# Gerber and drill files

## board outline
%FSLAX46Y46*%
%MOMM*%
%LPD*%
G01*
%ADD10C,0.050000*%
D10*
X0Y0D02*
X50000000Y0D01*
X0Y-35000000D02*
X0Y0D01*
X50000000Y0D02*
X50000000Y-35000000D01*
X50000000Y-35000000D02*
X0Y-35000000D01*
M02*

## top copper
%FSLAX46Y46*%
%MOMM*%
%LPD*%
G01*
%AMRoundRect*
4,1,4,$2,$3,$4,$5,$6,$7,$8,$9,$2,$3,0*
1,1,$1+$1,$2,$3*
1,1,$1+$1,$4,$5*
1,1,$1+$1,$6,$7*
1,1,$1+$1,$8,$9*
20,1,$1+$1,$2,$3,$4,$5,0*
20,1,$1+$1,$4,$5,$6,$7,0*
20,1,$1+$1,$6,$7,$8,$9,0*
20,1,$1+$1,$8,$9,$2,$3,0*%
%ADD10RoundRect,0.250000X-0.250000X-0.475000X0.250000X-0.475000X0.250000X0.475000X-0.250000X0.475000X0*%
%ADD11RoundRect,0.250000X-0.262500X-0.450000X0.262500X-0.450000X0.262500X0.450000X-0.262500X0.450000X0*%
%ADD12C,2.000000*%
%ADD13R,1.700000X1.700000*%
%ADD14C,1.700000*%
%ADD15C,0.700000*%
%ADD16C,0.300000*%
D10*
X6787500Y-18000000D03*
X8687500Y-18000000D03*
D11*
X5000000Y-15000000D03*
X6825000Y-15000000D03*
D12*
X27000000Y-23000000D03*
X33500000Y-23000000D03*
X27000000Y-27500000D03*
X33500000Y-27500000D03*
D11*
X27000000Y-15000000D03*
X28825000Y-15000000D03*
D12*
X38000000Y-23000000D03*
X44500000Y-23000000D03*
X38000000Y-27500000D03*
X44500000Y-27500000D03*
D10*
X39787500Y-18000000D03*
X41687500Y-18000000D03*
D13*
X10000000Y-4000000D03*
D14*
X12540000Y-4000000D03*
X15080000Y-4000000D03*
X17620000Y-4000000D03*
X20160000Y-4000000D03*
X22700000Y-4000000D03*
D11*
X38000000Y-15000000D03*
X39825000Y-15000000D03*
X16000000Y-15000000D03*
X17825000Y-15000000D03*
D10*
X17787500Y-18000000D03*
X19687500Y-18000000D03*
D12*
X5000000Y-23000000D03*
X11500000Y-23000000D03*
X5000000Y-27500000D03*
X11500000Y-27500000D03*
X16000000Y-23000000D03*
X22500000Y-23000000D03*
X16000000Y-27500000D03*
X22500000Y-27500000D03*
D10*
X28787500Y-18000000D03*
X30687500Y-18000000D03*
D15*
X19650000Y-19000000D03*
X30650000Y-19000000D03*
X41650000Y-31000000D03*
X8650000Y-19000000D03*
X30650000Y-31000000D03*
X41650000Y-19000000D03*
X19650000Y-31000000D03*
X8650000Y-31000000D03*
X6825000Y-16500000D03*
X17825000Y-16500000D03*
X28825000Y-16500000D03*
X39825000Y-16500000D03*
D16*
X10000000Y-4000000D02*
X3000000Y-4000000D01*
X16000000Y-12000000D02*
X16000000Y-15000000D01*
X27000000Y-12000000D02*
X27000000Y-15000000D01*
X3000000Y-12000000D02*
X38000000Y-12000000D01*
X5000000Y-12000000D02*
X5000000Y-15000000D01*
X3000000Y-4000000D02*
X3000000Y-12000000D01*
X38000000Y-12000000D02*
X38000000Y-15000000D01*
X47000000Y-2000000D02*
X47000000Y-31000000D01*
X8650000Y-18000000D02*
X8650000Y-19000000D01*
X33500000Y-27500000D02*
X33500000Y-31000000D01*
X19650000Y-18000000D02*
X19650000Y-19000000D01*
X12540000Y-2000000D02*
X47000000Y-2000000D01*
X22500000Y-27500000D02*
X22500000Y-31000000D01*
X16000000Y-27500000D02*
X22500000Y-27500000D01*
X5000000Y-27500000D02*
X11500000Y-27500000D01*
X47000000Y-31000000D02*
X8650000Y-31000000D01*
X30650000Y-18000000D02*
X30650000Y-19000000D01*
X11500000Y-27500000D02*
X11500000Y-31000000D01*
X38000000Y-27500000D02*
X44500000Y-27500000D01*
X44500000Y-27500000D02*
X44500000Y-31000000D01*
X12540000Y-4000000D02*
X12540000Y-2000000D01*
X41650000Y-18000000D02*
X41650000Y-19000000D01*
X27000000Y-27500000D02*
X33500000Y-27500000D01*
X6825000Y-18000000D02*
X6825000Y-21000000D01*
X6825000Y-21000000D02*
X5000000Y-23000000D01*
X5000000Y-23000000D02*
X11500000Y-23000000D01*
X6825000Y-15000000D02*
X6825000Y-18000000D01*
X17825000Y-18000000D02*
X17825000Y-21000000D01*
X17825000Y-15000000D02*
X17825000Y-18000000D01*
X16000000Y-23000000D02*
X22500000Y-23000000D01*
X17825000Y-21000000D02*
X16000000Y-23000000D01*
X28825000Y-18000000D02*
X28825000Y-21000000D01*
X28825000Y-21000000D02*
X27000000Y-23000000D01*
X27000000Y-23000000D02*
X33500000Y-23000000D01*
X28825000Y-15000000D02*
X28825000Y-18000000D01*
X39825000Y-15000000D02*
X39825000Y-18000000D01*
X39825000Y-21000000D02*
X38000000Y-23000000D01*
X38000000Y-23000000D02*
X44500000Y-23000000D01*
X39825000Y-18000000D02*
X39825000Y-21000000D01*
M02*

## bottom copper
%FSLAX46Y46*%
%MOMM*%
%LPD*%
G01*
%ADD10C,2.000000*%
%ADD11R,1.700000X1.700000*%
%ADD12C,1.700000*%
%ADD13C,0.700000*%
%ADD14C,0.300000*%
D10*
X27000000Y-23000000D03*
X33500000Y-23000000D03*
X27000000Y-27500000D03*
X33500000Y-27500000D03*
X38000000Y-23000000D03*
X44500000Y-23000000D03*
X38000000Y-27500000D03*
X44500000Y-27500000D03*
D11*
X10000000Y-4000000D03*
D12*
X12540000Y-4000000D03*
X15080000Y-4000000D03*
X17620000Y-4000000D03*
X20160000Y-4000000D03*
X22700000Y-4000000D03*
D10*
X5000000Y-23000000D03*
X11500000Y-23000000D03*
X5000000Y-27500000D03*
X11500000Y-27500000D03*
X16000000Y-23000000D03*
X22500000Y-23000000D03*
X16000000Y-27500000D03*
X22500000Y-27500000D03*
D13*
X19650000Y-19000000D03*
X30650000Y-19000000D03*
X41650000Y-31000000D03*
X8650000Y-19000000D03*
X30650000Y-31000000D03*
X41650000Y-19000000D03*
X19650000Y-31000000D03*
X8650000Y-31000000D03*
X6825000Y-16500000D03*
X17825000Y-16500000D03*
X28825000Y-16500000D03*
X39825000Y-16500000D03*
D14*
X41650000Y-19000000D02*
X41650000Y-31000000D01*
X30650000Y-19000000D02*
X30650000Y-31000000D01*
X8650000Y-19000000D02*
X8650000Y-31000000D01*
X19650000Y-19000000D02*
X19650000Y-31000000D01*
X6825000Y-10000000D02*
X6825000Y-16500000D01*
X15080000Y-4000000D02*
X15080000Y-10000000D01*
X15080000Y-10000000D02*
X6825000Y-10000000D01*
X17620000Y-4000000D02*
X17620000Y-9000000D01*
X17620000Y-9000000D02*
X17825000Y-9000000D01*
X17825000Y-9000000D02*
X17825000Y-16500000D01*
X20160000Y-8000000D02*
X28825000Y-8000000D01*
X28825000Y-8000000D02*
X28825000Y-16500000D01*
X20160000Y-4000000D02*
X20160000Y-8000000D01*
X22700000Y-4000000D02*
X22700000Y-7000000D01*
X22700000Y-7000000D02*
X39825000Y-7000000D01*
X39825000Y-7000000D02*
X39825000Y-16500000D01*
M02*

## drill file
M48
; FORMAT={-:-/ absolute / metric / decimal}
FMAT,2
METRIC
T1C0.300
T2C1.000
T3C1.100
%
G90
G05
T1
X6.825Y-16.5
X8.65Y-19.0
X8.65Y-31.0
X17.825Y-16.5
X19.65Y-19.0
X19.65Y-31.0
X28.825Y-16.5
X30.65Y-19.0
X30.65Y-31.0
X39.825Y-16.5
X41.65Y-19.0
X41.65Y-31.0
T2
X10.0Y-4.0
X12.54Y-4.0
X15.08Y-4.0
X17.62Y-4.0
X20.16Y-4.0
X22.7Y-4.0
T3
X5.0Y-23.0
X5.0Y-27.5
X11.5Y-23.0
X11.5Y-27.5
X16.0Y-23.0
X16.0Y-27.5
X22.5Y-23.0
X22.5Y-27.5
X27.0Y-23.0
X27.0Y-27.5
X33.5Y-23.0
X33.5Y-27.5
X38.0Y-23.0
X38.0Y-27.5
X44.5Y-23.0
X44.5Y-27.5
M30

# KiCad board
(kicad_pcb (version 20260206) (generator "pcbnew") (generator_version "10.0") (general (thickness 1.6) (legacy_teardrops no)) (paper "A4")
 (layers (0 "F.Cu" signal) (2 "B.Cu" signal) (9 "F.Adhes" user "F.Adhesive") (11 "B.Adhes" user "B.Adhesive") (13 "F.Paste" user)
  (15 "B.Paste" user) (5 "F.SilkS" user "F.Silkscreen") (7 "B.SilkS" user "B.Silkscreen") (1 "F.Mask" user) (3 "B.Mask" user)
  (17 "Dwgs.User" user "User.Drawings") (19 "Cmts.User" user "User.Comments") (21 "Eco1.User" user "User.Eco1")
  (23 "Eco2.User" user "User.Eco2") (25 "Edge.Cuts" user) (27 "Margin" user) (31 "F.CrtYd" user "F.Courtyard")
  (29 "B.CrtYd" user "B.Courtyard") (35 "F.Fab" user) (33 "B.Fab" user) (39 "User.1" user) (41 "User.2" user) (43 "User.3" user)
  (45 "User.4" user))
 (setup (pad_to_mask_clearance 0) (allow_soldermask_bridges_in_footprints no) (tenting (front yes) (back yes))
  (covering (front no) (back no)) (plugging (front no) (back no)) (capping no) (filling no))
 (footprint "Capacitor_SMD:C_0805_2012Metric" (layer "F.Cu") (at 7.7375 18)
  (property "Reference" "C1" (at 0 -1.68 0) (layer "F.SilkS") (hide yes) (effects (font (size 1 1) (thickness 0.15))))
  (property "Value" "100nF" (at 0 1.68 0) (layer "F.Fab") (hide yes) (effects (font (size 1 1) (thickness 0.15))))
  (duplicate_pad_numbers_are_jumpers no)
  (pad "1" smd roundrect (at -0.95 0) (size 1 1.45) (layers "F.Cu" "F.Mask" "F.Paste") (roundrect_rratio 0.25) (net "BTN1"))
  (pad "2" smd roundrect (at 0.95 0) (size 1 1.45) (layers "F.Cu" "F.Mask" "F.Paste") (roundrect_rratio 0.25) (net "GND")))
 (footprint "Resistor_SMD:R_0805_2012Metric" (layer "F.Cu") (at 5.9125 15)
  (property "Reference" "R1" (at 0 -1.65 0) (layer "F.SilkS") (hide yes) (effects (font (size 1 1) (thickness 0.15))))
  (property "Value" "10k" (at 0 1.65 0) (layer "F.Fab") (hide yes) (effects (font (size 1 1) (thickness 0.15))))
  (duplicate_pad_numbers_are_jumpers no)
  (pad "1" smd roundrect (at -0.9125 0) (size 1.025 1.4) (layers "F.Cu" "F.Mask" "F.Paste") (roundrect_rratio 0.243902) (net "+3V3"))
  (pad "2" smd roundrect (at 0.9125 0) (size 1.025 1.4) (layers "F.Cu" "F.Mask" "F.Paste") (roundrect_rratio 0.243902) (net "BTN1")))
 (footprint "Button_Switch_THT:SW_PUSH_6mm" (layer "F.Cu") (at 27 23)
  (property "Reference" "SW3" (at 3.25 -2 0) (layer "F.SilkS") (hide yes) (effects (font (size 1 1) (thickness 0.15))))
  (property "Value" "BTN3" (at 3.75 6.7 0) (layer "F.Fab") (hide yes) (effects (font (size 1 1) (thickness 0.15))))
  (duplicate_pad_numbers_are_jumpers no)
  (pad "1" thru_hole circle (at 0 0 90) (size 2 2) (drill 1.1) (layers "*.Cu" "*.Mask") (remove_unused_layers no) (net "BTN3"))
  (pad "1" thru_hole circle (at 6.5 0 90) (size 2 2) (drill 1.1) (layers "*.Cu" "*.Mask") (remove_unused_layers no) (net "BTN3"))
  (pad "2" thru_hole circle (at 0 4.5 90) (size 2 2) (drill 1.1) (layers "*.Cu" "*.Mask") (remove_unused_layers no) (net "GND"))
  (pad "2" thru_hole circle (at 6.5 4.5 90) (size 2 2) (drill 1.1) (layers "*.Cu" "*.Mask") (remove_unused_layers no) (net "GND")))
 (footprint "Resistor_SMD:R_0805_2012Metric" (layer "F.Cu") (at 27.9125 15)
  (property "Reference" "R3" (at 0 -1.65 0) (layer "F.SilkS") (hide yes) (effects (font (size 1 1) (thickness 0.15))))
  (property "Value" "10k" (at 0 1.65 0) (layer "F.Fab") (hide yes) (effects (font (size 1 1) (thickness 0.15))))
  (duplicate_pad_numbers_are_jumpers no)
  (pad "1" smd roundrect (at -0.9125 0) (size 1.025 1.4) (layers "F.Cu" "F.Mask" "F.Paste") (roundrect_rratio 0.243902) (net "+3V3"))
  (pad "2" smd roundrect (at 0.9125 0) (size 1.025 1.4) (layers "F.Cu" "F.Mask" "F.Paste") (roundrect_rratio 0.243902) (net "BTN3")))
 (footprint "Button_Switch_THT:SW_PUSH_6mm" (layer "F.Cu") (at 38 23)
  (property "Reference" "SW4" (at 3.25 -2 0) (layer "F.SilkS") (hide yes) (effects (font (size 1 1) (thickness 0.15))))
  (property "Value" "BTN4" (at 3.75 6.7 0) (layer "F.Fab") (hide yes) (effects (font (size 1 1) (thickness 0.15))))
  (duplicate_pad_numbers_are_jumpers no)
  (pad "1" thru_hole circle (at 0 0 90) (size 2 2) (drill 1.1) (layers "*.Cu" "*.Mask") (remove_unused_layers no) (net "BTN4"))
  (pad "1" thru_hole circle (at 6.5 0 90) (size 2 2) (drill 1.1) (layers "*.Cu" "*.Mask") (remove_unused_layers no) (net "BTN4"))
  (pad "2" thru_hole circle (at 0 4.5 90) (size 2 2) (drill 1.1) (layers "*.Cu" "*.Mask") (remove_unused_layers no) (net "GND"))
  (pad "2" thru_hole circle (at 6.5 4.5 90) (size 2 2) (drill 1.1) (layers "*.Cu" "*.Mask") (remove_unused_layers no) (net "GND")))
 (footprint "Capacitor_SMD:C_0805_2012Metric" (layer "F.Cu") (at 40.7375 18)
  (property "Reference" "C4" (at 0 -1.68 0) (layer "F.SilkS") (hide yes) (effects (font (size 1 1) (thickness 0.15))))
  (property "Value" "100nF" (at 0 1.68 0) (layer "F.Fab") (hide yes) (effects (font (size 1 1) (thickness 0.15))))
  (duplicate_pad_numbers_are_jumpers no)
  (pad "1" smd roundrect (at -0.95 0) (size 1 1.45) (layers "F.Cu" "F.Mask" "F.Paste") (roundrect_rratio 0.25) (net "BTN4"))
  (pad "2" smd roundrect (at 0.95 0) (size 1 1.45) (layers "F.Cu" "F.Mask" "F.Paste") (roundrect_rratio 0.25) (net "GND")))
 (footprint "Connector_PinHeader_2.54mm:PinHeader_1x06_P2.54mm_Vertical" (layer "F.Cu") (at 10 4 90)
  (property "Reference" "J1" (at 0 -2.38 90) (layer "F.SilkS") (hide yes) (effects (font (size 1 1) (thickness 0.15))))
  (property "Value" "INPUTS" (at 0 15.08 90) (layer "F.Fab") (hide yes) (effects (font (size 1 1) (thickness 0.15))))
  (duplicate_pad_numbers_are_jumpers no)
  (pad "1" thru_hole rect (at 0 0 90) (size 1.7 1.7) (drill 1) (layers "*.Cu" "*.Mask") (remove_unused_layers no) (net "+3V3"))
  (pad "2" thru_hole circle (at 0 2.54 90) (size 1.7 1.7) (drill 1) (layers "*.Cu" "*.Mask") (remove_unused_layers no) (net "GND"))
  (pad "3" thru_hole circle (at 0 5.08 90) (size 1.7 1.7) (drill 1) (layers "*.Cu" "*.Mask") (remove_unused_layers no) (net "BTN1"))
  (pad "4" thru_hole circle (at 0 7.62 90) (size 1.7 1.7) (drill 1) (layers "*.Cu" "*.Mask") (remove_unused_layers no) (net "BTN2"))
  (pad "5" thru_hole circle (at 0 10.16 90) (size 1.7 1.7) (drill 1) (layers "*.Cu" "*.Mask") (remove_unused_layers no) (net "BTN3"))
  (pad "6" thru_hole circle (at 0 12.7 90) (size 1.7 1.7) (drill 1) (layers "*.Cu" "*.Mask") (remove_unused_layers no) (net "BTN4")))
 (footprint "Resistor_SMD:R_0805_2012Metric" (layer "F.Cu") (at 38.9125 15)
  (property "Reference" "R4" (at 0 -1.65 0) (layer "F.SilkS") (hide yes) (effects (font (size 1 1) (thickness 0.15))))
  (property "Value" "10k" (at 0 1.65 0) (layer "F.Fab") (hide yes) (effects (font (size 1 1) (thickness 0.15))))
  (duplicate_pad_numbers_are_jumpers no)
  (pad "1" smd roundrect (at -0.9125 0) (size 1.025 1.4) (layers "F.Cu" "F.Mask" "F.Paste") (roundrect_rratio 0.243902) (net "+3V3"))
  (pad "2" smd roundrect (at 0.9125 0) (size 1.025 1.4) (layers "F.Cu" "F.Mask" "F.Paste") (roundrect_rratio 0.243902) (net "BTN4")))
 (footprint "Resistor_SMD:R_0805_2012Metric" (layer "F.Cu") (at 16.9125 15)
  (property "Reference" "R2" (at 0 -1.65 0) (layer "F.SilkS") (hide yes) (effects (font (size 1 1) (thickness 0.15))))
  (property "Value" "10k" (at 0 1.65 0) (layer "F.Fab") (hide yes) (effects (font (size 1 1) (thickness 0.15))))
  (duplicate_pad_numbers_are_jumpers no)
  (pad "1" smd roundrect (at -0.9125 0) (size 1.025 1.4) (layers "F.Cu" "F.Mask" "F.Paste") (roundrect_rratio 0.243902) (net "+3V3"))
  (pad "2" smd roundrect (at 0.9125 0) (size 1.025 1.4) (layers "F.Cu" "F.Mask" "F.Paste") (roundrect_rratio 0.243902) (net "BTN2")))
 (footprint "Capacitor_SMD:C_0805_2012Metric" (layer "F.Cu") (at 18.7375 18)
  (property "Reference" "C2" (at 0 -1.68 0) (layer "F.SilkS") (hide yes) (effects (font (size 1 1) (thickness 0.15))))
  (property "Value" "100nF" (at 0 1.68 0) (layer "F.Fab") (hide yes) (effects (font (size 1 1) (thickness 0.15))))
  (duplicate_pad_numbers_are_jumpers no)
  (pad "1" smd roundrect (at -0.95 0) (size 1 1.45) (layers "F.Cu" "F.Mask" "F.Paste") (roundrect_rratio 0.25) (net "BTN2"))
  (pad "2" smd roundrect (at 0.95 0) (size 1 1.45) (layers "F.Cu" "F.Mask" "F.Paste") (roundrect_rratio 0.25) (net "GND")))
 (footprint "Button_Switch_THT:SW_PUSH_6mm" (layer "F.Cu") (at 5 23)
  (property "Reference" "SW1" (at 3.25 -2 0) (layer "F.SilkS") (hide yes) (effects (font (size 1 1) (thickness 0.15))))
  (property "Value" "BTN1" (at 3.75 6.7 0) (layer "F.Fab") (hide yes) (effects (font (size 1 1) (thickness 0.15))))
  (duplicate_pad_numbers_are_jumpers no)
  (pad "1" thru_hole circle (at 0 0 90) (size 2 2) (drill 1.1) (layers "*.Cu" "*.Mask") (remove_unused_layers no) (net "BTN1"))
  (pad "1" thru_hole circle (at 6.5 0 90) (size 2 2) (drill 1.1) (layers "*.Cu" "*.Mask") (remove_unused_layers no) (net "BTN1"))
  (pad "2" thru_hole circle (at 0 4.5 90) (size 2 2) (drill 1.1) (layers "*.Cu" "*.Mask") (remove_unused_layers no) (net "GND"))
  (pad "2" thru_hole circle (at 6.5 4.5 90) (size 2 2) (drill 1.1) (layers "*.Cu" "*.Mask") (remove_unused_layers no) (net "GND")))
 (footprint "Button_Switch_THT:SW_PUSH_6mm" (layer "F.Cu") (at 16 23)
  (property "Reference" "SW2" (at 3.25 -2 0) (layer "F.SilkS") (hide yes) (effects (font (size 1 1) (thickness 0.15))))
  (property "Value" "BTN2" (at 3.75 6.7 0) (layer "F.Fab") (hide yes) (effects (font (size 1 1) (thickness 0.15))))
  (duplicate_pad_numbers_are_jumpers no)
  (pad "1" thru_hole circle (at 0 0 90) (size 2 2) (drill 1.1) (layers "*.Cu" "*.Mask") (remove_unused_layers no) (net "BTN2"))
  (pad "1" thru_hole circle (at 6.5 0 90) (size 2 2) (drill 1.1) (layers "*.Cu" "*.Mask") (remove_unused_layers no) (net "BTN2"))
  (pad "2" thru_hole circle (at 0 4.5 90) (size 2 2) (drill 1.1) (layers "*.Cu" "*.Mask") (remove_unused_layers no) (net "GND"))
  (pad "2" thru_hole circle (at 6.5 4.5 90) (size 2 2) (drill 1.1) (layers "*.Cu" "*.Mask") (remove_unused_layers no) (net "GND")))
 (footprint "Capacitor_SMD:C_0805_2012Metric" (layer "F.Cu") (at 29.7375 18)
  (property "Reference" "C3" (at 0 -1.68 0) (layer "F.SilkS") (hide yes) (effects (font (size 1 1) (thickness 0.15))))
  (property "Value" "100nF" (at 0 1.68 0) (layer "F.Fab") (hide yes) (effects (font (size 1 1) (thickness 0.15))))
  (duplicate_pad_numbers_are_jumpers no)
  (pad "1" smd roundrect (at -0.95 0) (size 1 1.45) (layers "F.Cu" "F.Mask" "F.Paste") (roundrect_rratio 0.25) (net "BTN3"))
  (pad "2" smd roundrect (at 0.95 0) (size 1 1.45) (layers "F.Cu" "F.Mask" "F.Paste") (roundrect_rratio 0.25) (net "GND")))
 (gr_line (start 0 0) (end 50 0) (stroke (width 0.05) (type default)) (layer "Edge.Cuts"))
 (gr_line (start 0 35) (end 0 0) (stroke (width 0.05) (type default)) (layer "Edge.Cuts"))
 (gr_line (start 50 0) (end 50 35) (stroke (width 0.05) (type default)) (layer "Edge.Cuts"))
 (gr_line (start 50 35) (end 0 35) (stroke (width 0.05) (type default)) (layer "Edge.Cuts"))
 (segment (start 10 4) (end 3 4) (width 0.3) (layer "F.Cu") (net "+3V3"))
 (segment (start 16 12) (end 16 15) (width 0.3) (layer "F.Cu") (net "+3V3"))
 (segment (start 27 12) (end 27 15) (width 0.3) (layer "F.Cu") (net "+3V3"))
 (segment (start 3 12) (end 38 12) (width 0.3) (layer "F.Cu") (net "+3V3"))
 (segment (start 5 12) (end 5 15) (width 0.3) (layer "F.Cu") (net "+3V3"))
 (segment (start 3 4) (end 3 12) (width 0.3) (layer "F.Cu") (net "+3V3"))
 (segment (start 38 12) (end 38 15) (width 0.3) (layer "F.Cu") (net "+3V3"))
 (segment (start 47 2) (end 47 31) (width 0.3) (layer "F.Cu") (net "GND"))
 (segment (start 8.65 18) (end 8.65 19) (width 0.3) (layer "F.Cu") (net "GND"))
 (segment (start 33.5 27.5) (end 33.5 31) (width 0.3) (layer "F.Cu") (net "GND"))
 (segment (start 19.65 18) (end 19.65 19) (width 0.3) (layer "F.Cu") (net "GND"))
 (segment (start 12.54 2) (end 47 2) (width 0.3) (layer "F.Cu") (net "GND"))
 (segment (start 22.5 27.5) (end 22.5 31) (width 0.3) (layer "F.Cu") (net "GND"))
 (segment (start 16 27.5) (end 22.5 27.5) (width 0.3) (layer "F.Cu") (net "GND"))
 (segment (start 5 27.5) (end 11.5 27.5) (width 0.3) (layer "F.Cu") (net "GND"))
 (segment (start 47 31) (end 8.65 31) (width 0.3) (layer "F.Cu") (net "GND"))
 (segment (start 30.65 18) (end 30.65 19) (width 0.3) (layer "F.Cu") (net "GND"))
 (segment (start 11.5 27.5) (end 11.5 31) (width 0.3) (layer "F.Cu") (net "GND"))
 (segment (start 38 27.5) (end 44.5 27.5) (width 0.3) (layer "F.Cu") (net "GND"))
 (segment (start 44.5 27.5) (end 44.5 31) (width 0.3) (layer "F.Cu") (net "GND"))
 (segment (start 12.54 4) (end 12.54 2) (width 0.3) (layer "F.Cu") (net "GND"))
 (segment (start 41.65 18) (end 41.65 19) (width 0.3) (layer "F.Cu") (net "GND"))
 (segment (start 27 27.5) (end 33.5 27.5) (width 0.3) (layer "F.Cu") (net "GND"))
 (via (at 19.65 19) (size 0.7) (drill 0.3) (layers "F.Cu" "B.Cu") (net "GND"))
 (via (at 30.65 19) (size 0.7) (drill 0.3) (layers "F.Cu" "B.Cu") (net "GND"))
 (via (at 41.65 31) (size 0.7) (drill 0.3) (layers "F.Cu" "B.Cu") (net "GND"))
 (via (at 8.65 19) (size 0.7) (drill 0.3) (layers "F.Cu" "B.Cu") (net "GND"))
 (via (at 30.65 31) (size 0.7) (drill 0.3) (layers "F.Cu" "B.Cu") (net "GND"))
 (via (at 41.65 19) (size 0.7) (drill 0.3) (layers "F.Cu" "B.Cu") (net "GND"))
 (via (at 19.65 31) (size 0.7) (drill 0.3) (layers "F.Cu" "B.Cu") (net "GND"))
 (via (at 8.65 31) (size 0.7) (drill 0.3) (layers "F.Cu" "B.Cu") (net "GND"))
 (segment (start 41.65 19) (end 41.65 31) (width 0.3) (layer "B.Cu") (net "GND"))
 (segment (start 30.65 19) (end 30.65 31) (width 0.3) (layer "B.Cu") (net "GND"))
 (segment (start 8.65 19) (end 8.65 31) (width 0.3) (layer "B.Cu") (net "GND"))
 (segment (start 19.65 19) (end 19.65 31) (width 0.3) (layer "B.Cu") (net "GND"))
 (segment (start 6.825 18) (end 6.825 21) (width 0.3) (layer "F.Cu") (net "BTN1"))
 (segment (start 6.825 21) (end 5 23) (width 0.3) (layer "F.Cu") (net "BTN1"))
 (segment (start 5 23) (end 11.5 23) (width 0.3) (layer "F.Cu") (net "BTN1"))
 (segment (start 6.825 15) (end 6.825 18) (width 0.3) (layer "F.Cu") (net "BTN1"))
 (via (at 6.825 16.5) (size 0.7) (drill 0.3) (layers "F.Cu" "B.Cu") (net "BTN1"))
 (segment (start 6.825 10) (end 6.825 16.5) (width 0.3) (layer "B.Cu") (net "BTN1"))
 (segment (start 15.08 4) (end 15.08 10) (width 0.3) (layer "B.Cu") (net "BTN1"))
 (segment (start 15.08 10) (end 6.825 10) (width 0.3) (layer "B.Cu") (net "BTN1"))
 (segment (start 17.825 18) (end 17.825 21) (width 0.3) (layer "F.Cu") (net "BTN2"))
 (segment (start 17.825 15) (end 17.825 18) (width 0.3) (layer "F.Cu") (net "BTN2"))
 (segment (start 16 23) (end 22.5 23) (width 0.3) (layer "F.Cu") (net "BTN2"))
 (segment (start 17.825 21) (end 16 23) (width 0.3) (layer "F.Cu") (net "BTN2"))
 (via (at 17.825 16.5) (size 0.7) (drill 0.3) (layers "F.Cu" "B.Cu") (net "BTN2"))
 (segment (start 17.62 4) (end 17.62 9) (width 0.3) (layer "B.Cu") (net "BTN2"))
 (segment (start 17.62 9) (end 17.825 9) (width 0.3) (layer "B.Cu") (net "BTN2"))
 (segment (start 17.825 9) (end 17.825 16.5) (width 0.3) (layer "B.Cu") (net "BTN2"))
 (segment (start 28.825 18) (end 28.825 21) (width 0.3) (layer "F.Cu") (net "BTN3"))
 (segment (start 28.825 21) (end 27 23) (width 0.3) (layer "F.Cu") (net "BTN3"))
 (segment (start 27 23) (end 33.5 23) (width 0.3) (layer "F.Cu") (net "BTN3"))
 (segment (start 28.825 15) (end 28.825 18) (width 0.3) (layer "F.Cu") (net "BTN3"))
 (via (at 28.825 16.5) (size 0.7) (drill 0.3) (layers "F.Cu" "B.Cu") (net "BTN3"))
 (segment (start 20.16 8) (end 28.825 8) (width 0.3) (layer "B.Cu") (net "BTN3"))
 (segment (start 28.825 8) (end 28.825 16.5) (width 0.3) (layer "B.Cu") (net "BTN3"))
 (segment (start 20.16 4) (end 20.16 8) (width 0.3) (layer "B.Cu") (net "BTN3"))
 (segment (start 39.825 15) (end 39.825 18) (width 0.3) (layer "F.Cu") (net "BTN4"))
 (segment (start 39.825 21) (end 38 23) (width 0.3) (layer "F.Cu") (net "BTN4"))
 (segment (start 38 23) (end 44.5 23) (width 0.3) (layer "F.Cu") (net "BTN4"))
 (segment (start 39.825 18) (end 39.825 21) (width 0.3) (layer "F.Cu") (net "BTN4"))
 (via (at 39.825 16.5) (size 0.7) (drill 0.3) (layers "F.Cu" "B.Cu") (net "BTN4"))
 (segment (start 22.7 4) (end 22.7 7) (width 0.3) (layer "B.Cu") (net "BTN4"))
 (segment (start 22.7 7) (end 39.825 7) (width 0.3) (layer "B.Cu") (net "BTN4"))
 (segment (start 39.825 7) (end 39.825 16.5) (width 0.3) (layer "B.Cu") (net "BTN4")))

